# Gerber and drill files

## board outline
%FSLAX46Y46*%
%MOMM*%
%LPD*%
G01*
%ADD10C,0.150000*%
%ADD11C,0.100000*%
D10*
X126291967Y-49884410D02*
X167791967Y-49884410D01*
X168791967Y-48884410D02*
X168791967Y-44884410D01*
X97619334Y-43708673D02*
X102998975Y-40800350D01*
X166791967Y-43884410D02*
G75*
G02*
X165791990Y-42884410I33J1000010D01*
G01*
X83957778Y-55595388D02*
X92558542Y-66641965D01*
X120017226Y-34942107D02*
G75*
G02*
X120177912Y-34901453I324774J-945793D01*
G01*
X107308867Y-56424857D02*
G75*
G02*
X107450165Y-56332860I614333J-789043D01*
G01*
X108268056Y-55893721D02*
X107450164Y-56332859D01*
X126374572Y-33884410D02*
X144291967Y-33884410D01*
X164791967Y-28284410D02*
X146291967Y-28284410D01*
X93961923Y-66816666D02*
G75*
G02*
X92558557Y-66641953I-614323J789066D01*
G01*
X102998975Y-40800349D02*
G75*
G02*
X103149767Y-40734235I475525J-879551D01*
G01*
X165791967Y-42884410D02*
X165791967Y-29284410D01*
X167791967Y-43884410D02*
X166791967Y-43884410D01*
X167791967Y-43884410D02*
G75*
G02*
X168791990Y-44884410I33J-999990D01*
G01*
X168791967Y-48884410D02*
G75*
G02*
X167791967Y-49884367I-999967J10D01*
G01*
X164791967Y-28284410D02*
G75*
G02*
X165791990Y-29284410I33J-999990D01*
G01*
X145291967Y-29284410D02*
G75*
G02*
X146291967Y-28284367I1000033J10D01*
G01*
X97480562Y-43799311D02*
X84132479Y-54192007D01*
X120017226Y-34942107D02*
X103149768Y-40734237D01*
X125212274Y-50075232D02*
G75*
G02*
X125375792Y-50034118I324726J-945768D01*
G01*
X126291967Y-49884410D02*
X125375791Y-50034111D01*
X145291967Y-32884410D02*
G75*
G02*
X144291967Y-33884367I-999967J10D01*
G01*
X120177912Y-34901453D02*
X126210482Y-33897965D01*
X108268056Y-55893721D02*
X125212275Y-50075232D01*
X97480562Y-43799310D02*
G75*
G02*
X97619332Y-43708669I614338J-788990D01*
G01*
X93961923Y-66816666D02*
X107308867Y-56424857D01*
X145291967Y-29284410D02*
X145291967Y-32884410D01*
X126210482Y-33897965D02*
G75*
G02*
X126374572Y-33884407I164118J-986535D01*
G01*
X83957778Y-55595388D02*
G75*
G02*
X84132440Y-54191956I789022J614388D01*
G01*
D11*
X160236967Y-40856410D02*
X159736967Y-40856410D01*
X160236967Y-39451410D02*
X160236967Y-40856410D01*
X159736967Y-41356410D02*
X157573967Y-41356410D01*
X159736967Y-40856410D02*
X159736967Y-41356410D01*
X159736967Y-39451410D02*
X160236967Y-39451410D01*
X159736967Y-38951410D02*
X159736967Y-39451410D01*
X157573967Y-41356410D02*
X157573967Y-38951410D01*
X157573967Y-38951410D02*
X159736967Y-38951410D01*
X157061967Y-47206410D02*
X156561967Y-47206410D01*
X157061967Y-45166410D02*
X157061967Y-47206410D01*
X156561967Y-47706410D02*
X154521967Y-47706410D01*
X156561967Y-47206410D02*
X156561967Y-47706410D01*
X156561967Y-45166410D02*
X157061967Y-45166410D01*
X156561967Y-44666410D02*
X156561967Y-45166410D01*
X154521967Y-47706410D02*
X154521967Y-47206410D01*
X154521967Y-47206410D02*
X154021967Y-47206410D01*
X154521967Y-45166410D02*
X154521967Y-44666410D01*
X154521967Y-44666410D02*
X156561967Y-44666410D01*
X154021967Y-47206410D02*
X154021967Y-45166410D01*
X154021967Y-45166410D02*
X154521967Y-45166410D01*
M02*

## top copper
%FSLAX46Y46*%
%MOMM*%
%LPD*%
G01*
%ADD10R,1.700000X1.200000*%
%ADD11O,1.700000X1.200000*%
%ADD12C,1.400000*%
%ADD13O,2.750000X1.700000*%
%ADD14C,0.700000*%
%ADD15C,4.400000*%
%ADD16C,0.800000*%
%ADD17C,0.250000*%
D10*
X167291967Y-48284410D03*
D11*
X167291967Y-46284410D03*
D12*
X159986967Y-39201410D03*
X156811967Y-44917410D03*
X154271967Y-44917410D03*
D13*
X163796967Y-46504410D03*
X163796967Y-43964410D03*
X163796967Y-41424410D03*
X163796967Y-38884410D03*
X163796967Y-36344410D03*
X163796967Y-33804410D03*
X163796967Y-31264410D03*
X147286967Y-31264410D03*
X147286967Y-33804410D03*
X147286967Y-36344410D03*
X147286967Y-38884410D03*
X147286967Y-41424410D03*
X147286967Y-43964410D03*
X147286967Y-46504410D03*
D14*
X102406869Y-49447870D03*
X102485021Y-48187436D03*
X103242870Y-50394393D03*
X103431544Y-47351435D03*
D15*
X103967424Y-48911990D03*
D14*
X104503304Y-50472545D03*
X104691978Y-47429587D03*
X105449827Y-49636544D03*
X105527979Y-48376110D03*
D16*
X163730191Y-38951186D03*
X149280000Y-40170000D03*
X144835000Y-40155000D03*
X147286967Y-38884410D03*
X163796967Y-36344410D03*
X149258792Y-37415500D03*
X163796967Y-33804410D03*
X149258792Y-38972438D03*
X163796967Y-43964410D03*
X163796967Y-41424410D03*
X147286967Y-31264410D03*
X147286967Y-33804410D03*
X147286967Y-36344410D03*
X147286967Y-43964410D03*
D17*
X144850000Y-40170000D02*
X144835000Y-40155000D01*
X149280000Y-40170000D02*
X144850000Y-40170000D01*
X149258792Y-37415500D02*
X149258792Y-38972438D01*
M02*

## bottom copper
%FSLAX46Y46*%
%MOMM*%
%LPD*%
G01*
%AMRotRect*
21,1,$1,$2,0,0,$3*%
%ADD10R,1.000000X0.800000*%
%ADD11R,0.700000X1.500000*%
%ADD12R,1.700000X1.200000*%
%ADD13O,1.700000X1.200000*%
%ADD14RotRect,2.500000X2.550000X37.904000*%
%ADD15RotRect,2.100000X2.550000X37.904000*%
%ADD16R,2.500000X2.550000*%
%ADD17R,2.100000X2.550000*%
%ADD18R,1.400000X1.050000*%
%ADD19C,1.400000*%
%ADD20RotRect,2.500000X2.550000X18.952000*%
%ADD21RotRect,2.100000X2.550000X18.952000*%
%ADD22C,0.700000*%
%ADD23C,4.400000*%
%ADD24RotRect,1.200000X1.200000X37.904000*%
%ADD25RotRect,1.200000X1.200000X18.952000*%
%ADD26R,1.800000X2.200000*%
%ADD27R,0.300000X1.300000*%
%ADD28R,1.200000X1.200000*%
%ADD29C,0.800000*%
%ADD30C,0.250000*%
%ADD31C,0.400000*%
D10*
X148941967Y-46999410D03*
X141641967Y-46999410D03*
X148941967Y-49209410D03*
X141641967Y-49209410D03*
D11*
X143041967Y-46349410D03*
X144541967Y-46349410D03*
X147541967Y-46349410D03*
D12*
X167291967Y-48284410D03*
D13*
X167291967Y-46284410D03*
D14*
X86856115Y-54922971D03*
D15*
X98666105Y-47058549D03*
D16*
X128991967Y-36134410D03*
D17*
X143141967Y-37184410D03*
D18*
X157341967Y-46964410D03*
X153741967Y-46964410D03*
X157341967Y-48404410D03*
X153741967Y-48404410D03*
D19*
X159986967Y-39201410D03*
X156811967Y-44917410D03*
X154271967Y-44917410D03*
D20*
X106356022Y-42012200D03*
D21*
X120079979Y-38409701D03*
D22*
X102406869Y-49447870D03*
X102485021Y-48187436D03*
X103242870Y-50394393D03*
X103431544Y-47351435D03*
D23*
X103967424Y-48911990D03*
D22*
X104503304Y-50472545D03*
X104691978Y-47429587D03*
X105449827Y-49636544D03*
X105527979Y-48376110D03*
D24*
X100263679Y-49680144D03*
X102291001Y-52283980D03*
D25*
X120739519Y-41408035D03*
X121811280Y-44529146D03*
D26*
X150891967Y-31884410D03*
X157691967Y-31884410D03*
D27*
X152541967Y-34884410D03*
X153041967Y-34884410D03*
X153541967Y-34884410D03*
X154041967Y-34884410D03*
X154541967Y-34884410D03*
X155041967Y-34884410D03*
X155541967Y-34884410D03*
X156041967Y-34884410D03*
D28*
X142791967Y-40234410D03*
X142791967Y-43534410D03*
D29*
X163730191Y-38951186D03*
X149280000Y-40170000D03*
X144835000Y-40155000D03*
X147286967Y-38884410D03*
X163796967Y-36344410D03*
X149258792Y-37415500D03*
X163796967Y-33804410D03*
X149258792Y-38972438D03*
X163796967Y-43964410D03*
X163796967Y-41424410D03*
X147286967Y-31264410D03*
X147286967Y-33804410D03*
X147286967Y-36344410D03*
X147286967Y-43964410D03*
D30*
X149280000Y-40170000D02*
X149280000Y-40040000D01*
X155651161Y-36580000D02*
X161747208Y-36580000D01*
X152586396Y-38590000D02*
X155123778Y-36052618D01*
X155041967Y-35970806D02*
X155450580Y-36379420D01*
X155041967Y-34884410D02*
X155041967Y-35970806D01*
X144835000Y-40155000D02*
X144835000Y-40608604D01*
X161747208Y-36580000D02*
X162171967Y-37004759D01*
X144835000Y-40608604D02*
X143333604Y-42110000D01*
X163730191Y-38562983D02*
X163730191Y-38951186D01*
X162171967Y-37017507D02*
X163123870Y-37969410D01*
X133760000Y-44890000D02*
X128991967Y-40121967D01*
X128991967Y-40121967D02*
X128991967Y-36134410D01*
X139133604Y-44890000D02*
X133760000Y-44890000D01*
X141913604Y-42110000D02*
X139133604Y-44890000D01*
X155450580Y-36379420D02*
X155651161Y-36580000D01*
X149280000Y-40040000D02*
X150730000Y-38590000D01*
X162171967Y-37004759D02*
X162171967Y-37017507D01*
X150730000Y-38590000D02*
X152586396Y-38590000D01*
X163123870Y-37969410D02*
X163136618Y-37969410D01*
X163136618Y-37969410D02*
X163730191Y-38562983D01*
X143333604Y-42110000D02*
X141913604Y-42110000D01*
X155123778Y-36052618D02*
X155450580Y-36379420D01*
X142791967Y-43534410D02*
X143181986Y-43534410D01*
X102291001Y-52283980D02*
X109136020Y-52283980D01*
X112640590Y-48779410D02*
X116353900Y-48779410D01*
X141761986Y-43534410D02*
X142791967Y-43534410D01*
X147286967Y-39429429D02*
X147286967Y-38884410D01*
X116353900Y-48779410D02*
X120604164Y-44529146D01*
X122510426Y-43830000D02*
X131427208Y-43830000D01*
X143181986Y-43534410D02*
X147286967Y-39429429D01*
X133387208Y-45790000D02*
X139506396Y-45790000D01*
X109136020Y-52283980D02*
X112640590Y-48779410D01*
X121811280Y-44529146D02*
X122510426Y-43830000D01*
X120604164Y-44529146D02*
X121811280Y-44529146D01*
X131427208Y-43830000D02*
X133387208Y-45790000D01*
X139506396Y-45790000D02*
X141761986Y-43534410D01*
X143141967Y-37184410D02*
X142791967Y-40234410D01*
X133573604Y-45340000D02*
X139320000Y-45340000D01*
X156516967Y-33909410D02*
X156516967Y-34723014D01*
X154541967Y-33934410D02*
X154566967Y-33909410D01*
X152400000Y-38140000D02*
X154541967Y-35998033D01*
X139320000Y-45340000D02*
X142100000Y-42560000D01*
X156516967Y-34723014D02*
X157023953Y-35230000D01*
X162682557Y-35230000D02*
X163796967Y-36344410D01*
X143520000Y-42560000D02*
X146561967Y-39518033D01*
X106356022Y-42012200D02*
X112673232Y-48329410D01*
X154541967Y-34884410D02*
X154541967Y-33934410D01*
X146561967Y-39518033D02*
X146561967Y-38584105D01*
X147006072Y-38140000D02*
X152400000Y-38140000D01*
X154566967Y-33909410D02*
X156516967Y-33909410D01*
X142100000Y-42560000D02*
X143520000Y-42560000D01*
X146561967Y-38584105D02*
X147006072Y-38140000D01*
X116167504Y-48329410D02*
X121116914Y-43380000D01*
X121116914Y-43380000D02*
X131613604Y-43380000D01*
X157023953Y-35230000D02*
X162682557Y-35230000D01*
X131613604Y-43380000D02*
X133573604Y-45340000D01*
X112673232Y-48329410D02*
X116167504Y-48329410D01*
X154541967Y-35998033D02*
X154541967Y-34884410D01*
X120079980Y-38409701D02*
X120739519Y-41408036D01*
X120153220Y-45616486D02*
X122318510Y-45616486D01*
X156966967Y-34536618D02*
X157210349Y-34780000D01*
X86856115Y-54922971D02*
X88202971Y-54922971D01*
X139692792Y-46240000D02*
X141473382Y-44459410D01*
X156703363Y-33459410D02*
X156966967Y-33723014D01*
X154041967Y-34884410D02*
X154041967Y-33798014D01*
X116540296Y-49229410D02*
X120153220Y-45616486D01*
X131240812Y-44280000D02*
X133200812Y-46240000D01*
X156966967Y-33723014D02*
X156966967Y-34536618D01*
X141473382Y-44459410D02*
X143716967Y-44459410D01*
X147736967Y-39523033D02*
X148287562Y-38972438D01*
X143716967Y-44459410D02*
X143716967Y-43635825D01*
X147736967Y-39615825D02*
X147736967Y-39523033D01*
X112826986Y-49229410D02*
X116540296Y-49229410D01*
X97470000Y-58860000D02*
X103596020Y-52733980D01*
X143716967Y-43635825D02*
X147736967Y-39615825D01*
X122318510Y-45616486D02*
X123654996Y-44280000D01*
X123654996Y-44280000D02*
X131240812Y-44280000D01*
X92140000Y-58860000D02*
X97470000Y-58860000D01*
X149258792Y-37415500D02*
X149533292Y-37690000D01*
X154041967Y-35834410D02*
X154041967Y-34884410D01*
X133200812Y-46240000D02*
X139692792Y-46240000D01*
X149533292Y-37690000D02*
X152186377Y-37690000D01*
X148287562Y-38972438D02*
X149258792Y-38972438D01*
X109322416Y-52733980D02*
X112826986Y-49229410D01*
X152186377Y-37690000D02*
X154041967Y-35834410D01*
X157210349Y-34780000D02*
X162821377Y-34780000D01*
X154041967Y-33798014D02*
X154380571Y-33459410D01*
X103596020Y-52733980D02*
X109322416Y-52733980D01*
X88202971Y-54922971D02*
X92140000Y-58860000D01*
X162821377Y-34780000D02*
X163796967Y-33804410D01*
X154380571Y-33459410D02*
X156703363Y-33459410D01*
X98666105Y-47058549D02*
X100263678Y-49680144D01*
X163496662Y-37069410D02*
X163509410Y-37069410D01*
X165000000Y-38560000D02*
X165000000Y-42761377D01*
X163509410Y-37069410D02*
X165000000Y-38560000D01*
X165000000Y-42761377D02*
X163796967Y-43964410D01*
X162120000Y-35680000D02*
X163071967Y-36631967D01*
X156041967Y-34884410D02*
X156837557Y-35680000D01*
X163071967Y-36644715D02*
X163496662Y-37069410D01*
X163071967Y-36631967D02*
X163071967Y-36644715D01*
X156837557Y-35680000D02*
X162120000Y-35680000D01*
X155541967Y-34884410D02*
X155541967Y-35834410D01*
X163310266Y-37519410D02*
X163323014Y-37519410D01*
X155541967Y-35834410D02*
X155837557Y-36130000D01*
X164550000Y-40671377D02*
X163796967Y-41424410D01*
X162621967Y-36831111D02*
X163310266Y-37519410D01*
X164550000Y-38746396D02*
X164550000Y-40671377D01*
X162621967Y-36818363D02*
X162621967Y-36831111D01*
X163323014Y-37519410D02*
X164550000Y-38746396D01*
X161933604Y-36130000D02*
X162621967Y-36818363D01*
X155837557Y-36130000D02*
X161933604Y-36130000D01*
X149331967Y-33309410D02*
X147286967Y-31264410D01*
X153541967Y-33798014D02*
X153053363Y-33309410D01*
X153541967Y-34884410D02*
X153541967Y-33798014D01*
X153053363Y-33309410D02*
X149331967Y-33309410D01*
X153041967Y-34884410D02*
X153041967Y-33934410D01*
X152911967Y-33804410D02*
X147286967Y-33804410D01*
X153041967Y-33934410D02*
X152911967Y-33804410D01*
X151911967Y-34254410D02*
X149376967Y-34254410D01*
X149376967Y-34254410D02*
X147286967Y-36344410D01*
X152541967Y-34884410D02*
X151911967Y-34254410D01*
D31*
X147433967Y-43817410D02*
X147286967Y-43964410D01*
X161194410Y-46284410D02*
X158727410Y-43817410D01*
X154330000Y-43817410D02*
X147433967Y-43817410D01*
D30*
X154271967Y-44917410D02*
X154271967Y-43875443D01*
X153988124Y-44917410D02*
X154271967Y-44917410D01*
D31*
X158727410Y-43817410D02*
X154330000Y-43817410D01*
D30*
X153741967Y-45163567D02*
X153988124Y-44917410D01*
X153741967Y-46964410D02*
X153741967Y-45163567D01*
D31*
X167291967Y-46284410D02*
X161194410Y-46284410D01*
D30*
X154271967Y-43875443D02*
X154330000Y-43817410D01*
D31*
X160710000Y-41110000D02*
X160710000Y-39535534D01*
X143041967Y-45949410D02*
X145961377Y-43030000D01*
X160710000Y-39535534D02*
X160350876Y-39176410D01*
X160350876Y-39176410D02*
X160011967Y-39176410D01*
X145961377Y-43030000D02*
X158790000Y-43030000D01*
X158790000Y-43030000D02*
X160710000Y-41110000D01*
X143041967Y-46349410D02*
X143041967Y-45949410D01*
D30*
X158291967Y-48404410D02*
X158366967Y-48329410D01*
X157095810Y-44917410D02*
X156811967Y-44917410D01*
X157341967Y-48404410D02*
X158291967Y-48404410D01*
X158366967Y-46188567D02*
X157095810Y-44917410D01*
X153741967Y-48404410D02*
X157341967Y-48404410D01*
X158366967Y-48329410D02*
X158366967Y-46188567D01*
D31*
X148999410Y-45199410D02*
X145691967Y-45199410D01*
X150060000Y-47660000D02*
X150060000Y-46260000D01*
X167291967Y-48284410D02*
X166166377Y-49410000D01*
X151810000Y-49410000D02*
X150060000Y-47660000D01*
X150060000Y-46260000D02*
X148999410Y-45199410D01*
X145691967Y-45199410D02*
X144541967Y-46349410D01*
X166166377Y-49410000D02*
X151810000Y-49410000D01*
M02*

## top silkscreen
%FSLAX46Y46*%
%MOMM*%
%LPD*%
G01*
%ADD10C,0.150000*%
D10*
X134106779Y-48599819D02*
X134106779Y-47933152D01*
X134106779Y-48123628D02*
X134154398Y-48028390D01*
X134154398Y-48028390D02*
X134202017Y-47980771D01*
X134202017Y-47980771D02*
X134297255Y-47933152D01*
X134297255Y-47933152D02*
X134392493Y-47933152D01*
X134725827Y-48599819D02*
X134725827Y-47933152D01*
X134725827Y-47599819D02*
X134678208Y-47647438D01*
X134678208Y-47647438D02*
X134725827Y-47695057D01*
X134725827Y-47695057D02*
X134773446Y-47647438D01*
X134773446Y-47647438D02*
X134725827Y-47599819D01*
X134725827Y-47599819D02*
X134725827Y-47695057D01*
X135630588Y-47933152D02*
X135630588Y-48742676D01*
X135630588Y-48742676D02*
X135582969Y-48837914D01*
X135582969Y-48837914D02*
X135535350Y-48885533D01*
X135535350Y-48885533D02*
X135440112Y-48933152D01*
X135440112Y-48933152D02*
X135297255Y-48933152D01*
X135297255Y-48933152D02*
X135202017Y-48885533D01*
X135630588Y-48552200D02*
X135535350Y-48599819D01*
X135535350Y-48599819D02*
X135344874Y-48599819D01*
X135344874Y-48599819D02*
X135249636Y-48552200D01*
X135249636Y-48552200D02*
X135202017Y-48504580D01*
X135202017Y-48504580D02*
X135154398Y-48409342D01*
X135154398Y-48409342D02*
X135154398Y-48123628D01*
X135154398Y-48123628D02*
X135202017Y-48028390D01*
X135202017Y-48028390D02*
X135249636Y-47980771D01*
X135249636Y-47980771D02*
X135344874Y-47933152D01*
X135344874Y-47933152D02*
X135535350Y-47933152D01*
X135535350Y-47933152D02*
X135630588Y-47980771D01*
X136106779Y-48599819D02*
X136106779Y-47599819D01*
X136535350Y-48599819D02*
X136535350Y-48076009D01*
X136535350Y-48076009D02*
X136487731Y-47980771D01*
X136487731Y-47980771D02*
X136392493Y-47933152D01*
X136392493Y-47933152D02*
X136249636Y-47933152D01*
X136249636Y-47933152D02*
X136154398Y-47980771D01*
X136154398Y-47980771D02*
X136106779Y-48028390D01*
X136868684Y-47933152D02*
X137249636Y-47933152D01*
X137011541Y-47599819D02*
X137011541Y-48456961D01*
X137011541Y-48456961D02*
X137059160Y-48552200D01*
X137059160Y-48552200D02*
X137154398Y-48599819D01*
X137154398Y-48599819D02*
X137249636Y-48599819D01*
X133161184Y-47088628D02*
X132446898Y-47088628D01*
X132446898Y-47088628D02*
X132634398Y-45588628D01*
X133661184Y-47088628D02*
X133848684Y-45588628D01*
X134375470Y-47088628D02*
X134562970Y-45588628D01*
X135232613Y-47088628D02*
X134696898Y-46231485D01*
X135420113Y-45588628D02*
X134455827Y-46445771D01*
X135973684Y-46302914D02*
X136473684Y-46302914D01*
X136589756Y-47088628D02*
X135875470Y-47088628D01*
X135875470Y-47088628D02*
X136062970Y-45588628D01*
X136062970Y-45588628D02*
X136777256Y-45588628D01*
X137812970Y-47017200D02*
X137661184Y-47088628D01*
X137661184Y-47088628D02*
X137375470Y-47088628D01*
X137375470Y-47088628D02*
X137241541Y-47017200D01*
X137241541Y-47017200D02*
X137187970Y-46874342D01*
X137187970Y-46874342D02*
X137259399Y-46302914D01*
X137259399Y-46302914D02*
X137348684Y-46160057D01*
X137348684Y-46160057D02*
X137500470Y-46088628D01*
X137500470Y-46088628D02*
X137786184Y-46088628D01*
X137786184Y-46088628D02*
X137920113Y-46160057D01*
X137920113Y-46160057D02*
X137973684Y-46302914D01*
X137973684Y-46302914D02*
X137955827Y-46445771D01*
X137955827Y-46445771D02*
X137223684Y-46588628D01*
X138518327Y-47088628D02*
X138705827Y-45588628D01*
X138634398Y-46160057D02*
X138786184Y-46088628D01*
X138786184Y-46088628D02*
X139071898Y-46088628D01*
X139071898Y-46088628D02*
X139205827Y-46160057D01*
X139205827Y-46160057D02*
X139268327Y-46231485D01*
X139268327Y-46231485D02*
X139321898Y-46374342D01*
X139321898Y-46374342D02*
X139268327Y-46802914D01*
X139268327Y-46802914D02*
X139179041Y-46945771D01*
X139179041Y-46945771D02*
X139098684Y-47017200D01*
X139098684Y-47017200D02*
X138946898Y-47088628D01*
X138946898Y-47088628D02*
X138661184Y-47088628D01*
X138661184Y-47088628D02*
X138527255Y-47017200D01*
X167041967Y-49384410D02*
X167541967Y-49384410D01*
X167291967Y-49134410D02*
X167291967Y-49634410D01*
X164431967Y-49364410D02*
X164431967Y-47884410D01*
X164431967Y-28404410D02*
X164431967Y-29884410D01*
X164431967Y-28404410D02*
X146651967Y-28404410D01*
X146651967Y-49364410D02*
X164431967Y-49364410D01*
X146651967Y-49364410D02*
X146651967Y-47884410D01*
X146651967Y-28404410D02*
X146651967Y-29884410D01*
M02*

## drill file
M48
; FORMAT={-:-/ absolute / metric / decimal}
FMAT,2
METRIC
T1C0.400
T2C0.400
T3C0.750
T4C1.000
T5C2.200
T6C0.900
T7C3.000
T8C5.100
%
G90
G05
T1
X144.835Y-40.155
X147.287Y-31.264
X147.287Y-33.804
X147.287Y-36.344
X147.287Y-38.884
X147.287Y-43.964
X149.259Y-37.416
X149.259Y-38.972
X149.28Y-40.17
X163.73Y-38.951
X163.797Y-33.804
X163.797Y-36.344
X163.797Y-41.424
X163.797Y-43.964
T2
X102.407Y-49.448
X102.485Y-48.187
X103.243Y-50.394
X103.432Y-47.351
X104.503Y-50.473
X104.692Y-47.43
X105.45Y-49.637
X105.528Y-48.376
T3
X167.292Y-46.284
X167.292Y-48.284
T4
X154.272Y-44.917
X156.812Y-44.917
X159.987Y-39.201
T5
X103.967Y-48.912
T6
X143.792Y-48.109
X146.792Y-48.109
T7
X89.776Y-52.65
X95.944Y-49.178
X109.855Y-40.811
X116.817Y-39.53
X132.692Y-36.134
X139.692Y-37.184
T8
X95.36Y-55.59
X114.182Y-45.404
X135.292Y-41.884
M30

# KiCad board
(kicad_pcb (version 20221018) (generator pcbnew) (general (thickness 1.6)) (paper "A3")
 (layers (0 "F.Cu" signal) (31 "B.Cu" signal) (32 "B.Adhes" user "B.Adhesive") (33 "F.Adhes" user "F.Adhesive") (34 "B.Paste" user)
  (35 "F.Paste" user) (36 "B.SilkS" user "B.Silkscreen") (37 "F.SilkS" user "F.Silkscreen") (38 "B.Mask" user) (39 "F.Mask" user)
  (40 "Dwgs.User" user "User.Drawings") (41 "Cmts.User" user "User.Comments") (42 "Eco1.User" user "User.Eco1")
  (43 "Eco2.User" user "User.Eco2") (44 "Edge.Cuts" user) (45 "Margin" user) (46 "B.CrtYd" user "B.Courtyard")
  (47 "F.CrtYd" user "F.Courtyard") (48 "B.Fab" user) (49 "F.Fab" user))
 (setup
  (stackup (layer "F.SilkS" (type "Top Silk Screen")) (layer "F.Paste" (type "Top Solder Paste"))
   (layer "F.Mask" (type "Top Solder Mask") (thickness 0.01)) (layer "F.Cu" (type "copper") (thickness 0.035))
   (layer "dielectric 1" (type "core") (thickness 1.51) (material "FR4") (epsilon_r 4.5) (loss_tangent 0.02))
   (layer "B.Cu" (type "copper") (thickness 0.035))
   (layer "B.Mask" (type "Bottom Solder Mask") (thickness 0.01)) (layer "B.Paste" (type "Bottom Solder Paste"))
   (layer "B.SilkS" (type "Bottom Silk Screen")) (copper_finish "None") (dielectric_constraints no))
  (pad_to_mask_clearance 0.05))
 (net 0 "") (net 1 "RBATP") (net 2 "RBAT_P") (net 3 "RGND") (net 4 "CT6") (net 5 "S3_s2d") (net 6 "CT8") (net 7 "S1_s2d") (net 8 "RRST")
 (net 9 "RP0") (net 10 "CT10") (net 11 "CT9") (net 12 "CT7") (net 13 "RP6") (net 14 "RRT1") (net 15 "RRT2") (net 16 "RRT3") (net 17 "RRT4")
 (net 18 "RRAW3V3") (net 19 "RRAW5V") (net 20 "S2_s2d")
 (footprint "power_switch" (layer "F.Cu") (at 145.291967 48.08441 -90)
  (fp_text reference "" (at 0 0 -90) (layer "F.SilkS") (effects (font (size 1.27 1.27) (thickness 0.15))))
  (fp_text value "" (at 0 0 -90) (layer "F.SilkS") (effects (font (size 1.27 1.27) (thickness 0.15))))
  (pad "" smd rect (at -1.085 -3.65 180) (size 1 0.8) (layers "B.Cu" "B.Paste" "B.Mask"))
  (pad "" smd rect (at -1.085 3.65 180) (size 1 0.8) (layers "B.Cu" "B.Paste" "B.Mask"))
  (pad "" np_thru_hole circle (at 0.025 -1.5) (size 0.9 0.9) (drill 0.9) (layers "*.Cu" "*.Mask"))
  (pad "" np_thru_hole circle (at 0.025 1.5) (size 0.9 0.9) (drill 0.9) (layers "*.Cu" "*.Mask"))
  (pad "" smd rect (at 1.125 -3.65 180) (size 1 0.8) (layers "B.Cu" "B.Paste" "B.Mask"))
  (pad "" smd rect (at 1.125 3.65 180) (size 1 0.8) (layers "B.Cu" "B.Paste" "B.Mask"))
  (pad "4" smd rect (at -1.735 2.25 180) (size 0.7 1.5) (layers "B.Cu" "B.Paste" "B.Mask") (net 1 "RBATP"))
  (pad "5" smd rect (at -1.735 0.75 180) (size 0.7 1.5) (layers "B.Cu" "B.Paste" "B.Mask") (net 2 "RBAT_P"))
  (pad "6" smd rect (at -1.735 -2.25 180) (size 0.7 1.5) (layers "B.Cu" "B.Paste" "B.Mask")))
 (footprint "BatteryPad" (layer "F.Cu") (at 167.291967 47.28441 90)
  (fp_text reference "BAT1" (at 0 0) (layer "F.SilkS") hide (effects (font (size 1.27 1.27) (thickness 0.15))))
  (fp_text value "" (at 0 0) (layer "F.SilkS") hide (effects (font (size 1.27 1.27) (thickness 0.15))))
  (fp_line (start -2.1 -0.25) (end -2.1 0.25) (stroke (width 0.15) (type solid)) (layer "F.SilkS"))
  (fp_line (start -1.85 0) (end -2.35 0) (stroke (width 0.15) (type solid)) (layer "F.SilkS"))
  (pad "1" thru_hole rect (at -1 0 90) (size 1.2 1.7) (drill 0.75) (layers "*.Cu" "*.Mask") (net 2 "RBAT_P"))
  (pad "2" thru_hole oval (at 1 0 90) (size 1.2 1.7) (drill 0.75) (layers "*.Cu" "*.Mask") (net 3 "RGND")))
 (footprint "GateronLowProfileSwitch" (layer "F.Cu") (at 95.359531 55.589614 37.904)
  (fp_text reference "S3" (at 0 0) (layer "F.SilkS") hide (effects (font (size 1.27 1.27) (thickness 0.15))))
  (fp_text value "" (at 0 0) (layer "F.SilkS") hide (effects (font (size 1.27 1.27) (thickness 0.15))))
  (pad "" np_thru_hole circle (at -2.6 -5.75) (size 3 3) (drill 3) (layers "*.Cu" "*.Mask"))
  (pad "" np_thru_hole circle (at 0 0) (size 5.1 5.1) (drill 5.1) (layers "*.Cu" "*.Mask"))
  (pad "" np_thru_hole circle (at 4.4 -4.7) (size 3 3) (drill 3) (layers "*.Cu" "*.Mask"))
  (pad "1" smd rect (at -6.3 -5.75 37.904) (size 2.5 2.55) (layers "B.Cu" "B.Paste" "B.Mask") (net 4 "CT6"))
  (pad "2" smd rect (at 7.85 -4.7 37.904) (size 2.1 2.55) (layers "B.Cu" "B.Paste" "B.Mask") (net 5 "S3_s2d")))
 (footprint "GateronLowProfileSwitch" (layer "F.Cu") (at 135.291967 41.88441)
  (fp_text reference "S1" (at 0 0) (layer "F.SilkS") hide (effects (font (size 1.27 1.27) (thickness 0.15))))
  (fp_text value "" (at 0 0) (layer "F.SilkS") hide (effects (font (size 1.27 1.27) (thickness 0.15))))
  (pad "" np_thru_hole circle (at -2.6 -5.75) (size 3 3) (drill 3) (layers "*.Cu" "*.Mask"))
  (pad "" np_thru_hole circle (at 0 0) (size 5.1 5.1) (drill 5.1) (layers "*.Cu" "*.Mask"))
  (pad "" np_thru_hole circle (at 4.4 -4.7) (size 3 3) (drill 3) (layers "*.Cu" "*.Mask"))
  (pad "1" smd rect (at -6.3 -5.75) (size 2.5 2.55) (layers "B.Cu" "B.Paste" "B.Mask") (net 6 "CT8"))
  (pad "2" smd rect (at 7.85 -4.7) (size 2.1 2.55) (layers "B.Cu" "B.Paste" "B.Mask") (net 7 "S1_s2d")))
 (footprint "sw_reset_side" (layer "F.Cu") (at 155.541967 47.68441 -90)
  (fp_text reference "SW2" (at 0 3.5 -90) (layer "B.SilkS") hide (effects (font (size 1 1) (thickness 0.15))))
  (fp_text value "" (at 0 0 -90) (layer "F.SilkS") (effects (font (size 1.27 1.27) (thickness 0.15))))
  (pad "1" smd rect (at -0.72 -1.8 180) (size 1.4 1.05) (layers "B.Cu" "B.Paste" "B.Mask") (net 3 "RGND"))
  (pad "1" smd rect (at -0.72 1.8 180) (size 1.4 1.05) (layers "B.Cu" "B.Paste" "B.Mask") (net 3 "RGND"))
  (pad "2" smd rect (at 0.72 -1.8 180) (size 1.4 1.05) (layers "B.Cu" "B.Paste" "B.Mask") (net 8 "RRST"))
  (pad "2" smd rect (at 0.72 1.8 180) (size 1.4 1.05) (layers "B.Cu" "B.Paste" "B.Mask") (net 8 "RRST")))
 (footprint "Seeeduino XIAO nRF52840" (layer "F.Cu") (at 155.541967 38.88441 180)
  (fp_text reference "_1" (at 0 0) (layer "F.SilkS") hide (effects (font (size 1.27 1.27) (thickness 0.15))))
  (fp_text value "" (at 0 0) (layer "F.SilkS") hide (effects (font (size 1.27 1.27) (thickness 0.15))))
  (fp_line (start -8.89 -10.48) (end -8.89 -9) (stroke (width 0.15) (type solid)) (layer "F.SilkS"))
  (fp_line (start -8.89 10.48) (end -8.89 9) (stroke (width 0.15) (type solid)) (layer "F.SilkS"))
  (fp_line (start -8.89 10.48) (end 8.89 10.48) (stroke (width 0.15) (type solid)) (layer "F.SilkS"))
  (fp_line (start 8.89 -10.48) (end -8.89 -10.48) (stroke (width 0.15) (type solid)) (layer "F.SilkS"))
  (fp_line (start 8.89 -10.48) (end 8.89 -9) (stroke (width 0.15) (type solid)) (layer "F.SilkS"))
  (fp_line (start 8.89 10.48) (end 8.89 9) (stroke (width 0.15) (type solid)) (layer "F.SilkS"))
  (fp_line (start -4.695 -1.972) (end -4.195 -1.972) (stroke (width 0.1) (type solid)) (layer "Edge.Cuts"))
  (fp_line (start -4.695 -0.567) (end -4.695 -1.972) (stroke (width 0.1) (type solid)) (layer "Edge.Cuts"))
  (fp_line (start -4.195 -2.472) (end -2.032 -2.472) (stroke (width 0.1) (type solid)) (layer "Edge.Cuts"))
  (fp_line (start -4.195 -1.972) (end -4.195 -2.472) (stroke (width 0.1) (type solid)) (layer "Edge.Cuts"))
  (fp_line (start -4.195 -0.567) (end -4.695 -0.567) (stroke (width 0.1) (type solid)) (layer "Edge.Cuts"))
  (fp_line (start -4.195 -0.067) (end -4.195 -0.567) (stroke (width 0.1) (type solid)) (layer "Edge.Cuts"))
  (fp_line (start -2.032 -2.472) (end -2.032 -0.067) (stroke (width 0.1) (type solid)) (layer "Edge.Cuts"))
  (fp_line (start -2.032 -0.067) (end -4.195 -0.067) (stroke (width 0.1) (type solid)) (layer "Edge.Cuts"))
  (fp_line (start -1.52 -8.322) (end -1.02 -8.322) (stroke (width 0.1) (type solid)) (layer "Edge.Cuts"))
  (fp_line (start -1.52 -6.282) (end -1.52 -8.322) (stroke (width 0.1) (type solid)) (layer "Edge.Cuts"))
  (fp_line (start -1.02 -8.822) (end 1.02 -8.822) (stroke (width 0.1) (type solid)) (layer "Edge.Cuts"))
  (fp_line (start -1.02 -8.322) (end -1.02 -8.822) (stroke (width 0.1) (type solid)) (layer "Edge.Cuts"))
  (fp_line (start -1.02 -6.282) (end -1.52 -6.282) (stroke (width 0.1) (type solid)) (layer "Edge.Cuts"))
  (fp_line (start -1.02 -5.782) (end -1.02 -6.282) (stroke (width 0.1) (type solid)) (layer "Edge.Cuts"))
  (fp_line (start 1.02 -8.822) (end 1.02 -8.322) (stroke (width 0.1) (type solid)) (layer "Edge.Cuts"))
  (fp_line (start 1.02 -8.322) (end 1.52 -8.322) (stroke (width 0.1) (type solid)) (layer "Edge.Cuts"))
  (fp_line (start 1.02 -6.282) (end 1.02 -5.782) (stroke (width 0.1) (type solid)) (layer "Edge.Cuts"))
  (fp_line (start 1.02 -5.782) (end -1.02 -5.782) (stroke (width 0.1) (type solid)) (layer "Edge.Cuts"))
  (fp_line (start 1.52 -8.322) (end 1.52 -6.282) (stroke (width 0.1) (type solid)) (layer "Edge.Cuts"))
  (fp_line (start 1.52 -6.282) (end 1.02 -6.282) (stroke (width 0.1) (type solid)) (layer "Edge.Cuts"))
  (pad "" thru_hole circle (at -4.445 -0.317) (size 1.4 1.4) (drill 1) (layers "*.Cu" "*.Mask") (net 1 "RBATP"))
  (pad "" thru_hole circle (at -1.27 -6.033) (size 1.4 1.4) (drill 1) (layers "*.Cu" "*.Mask") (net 8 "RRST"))
  (pad "" thru_hole circle (at 1.27 -6.033) (size 1.4 1.4) (drill 1) (layers "*.Cu" "*.Mask") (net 3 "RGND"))
  (pad "1" smd oval (at -8.255 -7.62 180) (size 2.75 1.7) (layers "F.Cu" "F.Paste" "F.Mask") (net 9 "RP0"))
  (pad "2" smd oval (at -8.255 -5.08 180) (size 2.75 1.7) (layers "F.Cu" "F.Paste" "F.Mask") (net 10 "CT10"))
  (pad "3" smd oval (at -8.255 -2.54 180) (size 2.75 1.7) (layers "F.Cu" "F.Paste" "F.Mask") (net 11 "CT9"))
  (pad "4" smd oval (at -8.255 0 180) (size 2.75 1.7) (layers "F.Cu" "F.Paste" "F.Mask") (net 6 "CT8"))
  (pad "5" smd oval (at -8.255 2.54 180) (size 2.75 1.7) (layers "F.Cu" "F.Paste" "F.Mask") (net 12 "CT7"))
  (pad "6" smd oval (at -8.255 5.08 180) (size 2.75 1.7) (layers "F.Cu" "F.Paste" "F.Mask") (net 4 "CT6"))
  (pad "7" smd oval (at -8.255 7.62 180) (size 2.75 1.7) (layers "F.Cu" "F.Paste" "F.Mask") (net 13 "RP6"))
  (pad "8" smd oval (at 8.255 7.62 180) (size 2.75 1.7) (layers "F.Cu" "F.Paste" "F.Mask") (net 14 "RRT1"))
  (pad "9" smd oval (at 8.255 5.08 180) (size 2.75 1.7) (layers "F.Cu" "F.Paste" "F.Mask") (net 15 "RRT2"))
  (pad "10" smd oval (at 8.255 2.54 180) (size 2.75 1.7) (layers "F.Cu" "F.Paste" "F.Mask") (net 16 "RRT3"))
  (pad "11" smd oval (at 8.255 0 180) (size 2.75 1.7) (layers "F.Cu" "F.Paste" "F.Mask") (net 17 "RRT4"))
  (pad "12" smd oval (at 8.255 -2.54 180) (size 2.75 1.7) (layers "F.Cu" "F.Paste" "F.Mask") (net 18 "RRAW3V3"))
  (pad "13" smd oval (at 8.255 -5.08 180) (size 2.75 1.7) (layers "F.Cu" "F.Paste" "F.Mask") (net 3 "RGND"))
  (pad "14" smd oval (at 8.255 -7.62 180) (size 2.75 1.7) (layers "F.Cu" "F.Paste" "F.Mask") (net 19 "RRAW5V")))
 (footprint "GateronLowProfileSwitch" (layer "F.Cu") (at 114.181967 45.40441 18.952)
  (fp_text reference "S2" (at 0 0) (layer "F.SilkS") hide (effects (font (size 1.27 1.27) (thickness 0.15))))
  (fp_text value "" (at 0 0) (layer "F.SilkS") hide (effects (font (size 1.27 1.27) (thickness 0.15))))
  (pad "" np_thru_hole circle (at -2.6 -5.75) (size 3 3) (drill 3) (layers "*.Cu" "*.Mask"))
  (pad "" np_thru_hole circle (at 0 0) (size 5.1 5.1) (drill 5.1) (layers "*.Cu" "*.Mask"))
  (pad "" np_thru_hole circle (at 4.4 -4.7) (size 3 3) (drill 3) (layers "*.Cu" "*.Mask"))
  (pad "1" smd rect (at -6.3 -5.75 18.952) (size 2.5 2.55) (layers "B.Cu" "B.Paste" "B.Mask") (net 12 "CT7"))
  (pad "2" smd rect (at 7.85 -4.7 18.952) (size 2.1 2.55) (layers "B.Cu" "B.Paste" "B.Mask") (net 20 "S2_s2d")))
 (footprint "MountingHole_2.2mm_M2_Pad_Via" (layer "F.Cu") (at 103.967424 48.91199 18.952)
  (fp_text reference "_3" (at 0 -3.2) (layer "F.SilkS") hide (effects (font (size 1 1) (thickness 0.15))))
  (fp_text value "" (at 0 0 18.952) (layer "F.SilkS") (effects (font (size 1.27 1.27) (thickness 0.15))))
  (pad "1" thru_hole circle (at -1.65 0) (size 0.7 0.7) (drill 0.4) (layers "*.Cu" "*.Mask"))
  (pad "1" thru_hole circle (at -1.166726 -1.166726) (size 0.7 0.7) (drill 0.4) (layers "*.Cu" "*.Mask"))
  (pad "1" thru_hole circle (at -1.166726 1.166726) (size 0.7 0.7) (drill 0.4) (layers "*.Cu" "*.Mask"))
  (pad "1" thru_hole circle (at 0 -1.65) (size 0.7 0.7) (drill 0.4) (layers "*.Cu" "*.Mask"))
  (pad "1" thru_hole circle (at 0 0) (size 4.4 4.4) (drill 2.2) (layers "*.Cu" "*.Mask"))
  (pad "1" thru_hole circle (at 0 1.65) (size 0.7 0.7) (drill 0.4) (layers "*.Cu" "*.Mask"))
  (pad "1" thru_hole circle (at 1.166726 -1.166726) (size 0.7 0.7) (drill 0.4) (layers "*.Cu" "*.Mask"))
  (pad "1" thru_hole circle (at 1.166726 1.166726) (size 0.7 0.7) (drill 0.4) (layers "*.Cu" "*.Mask"))
  (pad "1" thru_hole circle (at 1.65 0) (size 0.7 0.7) (drill 0.4) (layers "*.Cu" "*.Mask")))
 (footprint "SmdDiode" (layer "B.Cu") (at 95.359531 55.589614 37.904)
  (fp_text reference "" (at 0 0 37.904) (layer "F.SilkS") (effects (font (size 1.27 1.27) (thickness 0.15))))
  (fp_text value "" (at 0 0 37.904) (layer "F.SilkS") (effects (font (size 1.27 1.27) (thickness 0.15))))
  (pad "1" smd rect (at 7.5 -1.65 37.904) (size 1.2 1.2) (layers "B.Cu" "B.Paste" "B.Mask") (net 5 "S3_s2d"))
  (pad "2" smd rect (at 7.5 1.65 37.904) (size 1.2 1.2) (layers "B.Cu" "B.Paste" "B.Mask") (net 17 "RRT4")))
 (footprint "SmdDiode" (layer "B.Cu") (at 114.181967 45.40441 18.952)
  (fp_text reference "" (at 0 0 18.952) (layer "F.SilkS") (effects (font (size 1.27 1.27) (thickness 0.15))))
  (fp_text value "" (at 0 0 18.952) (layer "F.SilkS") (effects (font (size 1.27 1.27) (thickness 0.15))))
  (pad "1" smd rect (at 7.5 -1.65 18.952) (size 1.2 1.2) (layers "B.Cu" "B.Paste" "B.Mask") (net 20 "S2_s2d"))
  (pad "2" smd rect (at 7.5 1.65 18.952) (size 1.2 1.2) (layers "B.Cu" "B.Paste" "B.Mask") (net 17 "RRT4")))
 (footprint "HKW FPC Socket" (layer "B.Cu") (at 154.291967 31.88441)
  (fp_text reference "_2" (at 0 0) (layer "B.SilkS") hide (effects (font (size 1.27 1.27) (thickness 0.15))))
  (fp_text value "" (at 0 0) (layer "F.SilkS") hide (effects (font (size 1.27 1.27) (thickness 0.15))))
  (pad "" smd rect (at -3.4 0) (size 1.8 2.2) (layers "B.Cu" "B.Paste" "B.Mask"))
  (pad "" smd rect (at 3.4 0) (size 1.8 2.2) (layers "B.Cu" "B.Paste" "B.Mask"))
  (pad "1" smd rect (at -1.75 3) (size 0.3 1.3) (layers "B.Cu" "B.Paste" "B.Mask") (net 16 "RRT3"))
  (pad "2" smd rect (at -1.25 3) (size 0.3 1.3) (layers "B.Cu" "B.Paste" "B.Mask") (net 15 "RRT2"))
  (pad "3" smd rect (at -0.75 3) (size 0.3 1.3) (layers "B.Cu" "B.Paste" "B.Mask") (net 14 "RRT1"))
  (pad "4" smd rect (at -0.25 3) (size 0.3 1.3) (layers "B.Cu" "B.Paste" "B.Mask") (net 4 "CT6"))
  (pad "5" smd rect (at 0.25 3) (size 0.3 1.3) (layers "B.Cu" "B.Paste" "B.Mask") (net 12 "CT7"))
  (pad "6" smd rect (at 0.75 3) (size 0.3 1.3) (layers "B.Cu" "B.Paste" "B.Mask") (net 6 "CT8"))
  (pad "7" smd rect (at 1.25 3) (size 0.3 1.3) (layers "B.Cu" "B.Paste" "B.Mask") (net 11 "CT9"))
  (pad "8" smd rect (at 1.75 3) (size 0.3 1.3) (layers "B.Cu" "B.Paste" "B.Mask") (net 10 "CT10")))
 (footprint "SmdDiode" (layer "B.Cu") (at 135.291967 41.88441)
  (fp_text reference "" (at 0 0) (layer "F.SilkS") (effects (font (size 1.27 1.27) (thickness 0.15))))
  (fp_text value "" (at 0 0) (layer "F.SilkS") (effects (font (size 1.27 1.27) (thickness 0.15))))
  (pad "1" smd rect (at 7.5 -1.65) (size 1.2 1.2) (layers "B.Cu" "B.Paste" "B.Mask") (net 7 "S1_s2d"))
  (pad "2" smd rect (at 7.5 1.65) (size 1.2 1.2) (layers "B.Cu" "B.Paste" "B.Mask") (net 17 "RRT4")))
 (gr_line (start 126.291967 49.88441) (end 167.791967 49.88441) (stroke (width 0.15) (type solid)) (layer "Edge.Cuts"))
 (gr_line (start 168.791967 48.88441) (end 168.791967 44.88441) (stroke (width 0.15) (type solid)) (layer "Edge.Cuts"))
 (gr_line (start 97.619334 43.708673) (end 102.998975 40.80035) (stroke (width 0.15) (type solid)) (layer "Edge.Cuts"))
 (gr_arc (start 166.791967 43.88441) (mid 166.08486 43.591517) (end 165.791967 42.88441) (stroke (width 0.15) (type solid))
  (layer "Edge.Cuts"))
 (gr_line (start 83.957778 55.595388) (end 92.558542 66.641965) (stroke (width 0.15) (type solid)) (layer "Edge.Cuts"))
 (gr_arc (start 120.017226 34.942107) (mid 120.096725 34.918445) (end 120.177912 34.901453) (stroke (width 0.15) (type solid))
  (layer "Edge.Cuts"))
 (gr_arc (start 107.308867 56.424857) (mid 107.377573 56.375875) (end 107.450164 56.332859) (stroke (width 0.15) (type solid))
  (layer "Edge.Cuts"))
 (gr_line (start 108.268056 55.893721) (end 107.450164 56.332859) (stroke (width 0.15) (type solid)) (layer "Edge.Cuts"))
 (gr_line (start 126.374572 33.88441) (end 144.291967 33.88441) (stroke (width 0.15) (type solid)) (layer "Edge.Cuts"))
 (gr_line (start 164.791967 28.28441) (end 146.291967 28.28441) (stroke (width 0.15) (type solid)) (layer "Edge.Cuts"))
 (gr_arc (start 93.961923 66.816666) (mid 93.224051 67.019965) (end 92.558542 66.641965) (stroke (width 0.15) (type solid))
  (layer "Edge.Cuts"))
 (gr_arc (start 102.998975 40.800349) (mid 103.073008 40.764184) (end 103.149768 40.734237) (stroke (width 0.15) (type solid))
  (layer "Edge.Cuts"))
 (gr_line (start 165.791967 42.88441) (end 165.791967 29.28441) (stroke (width 0.15) (type solid)) (layer "Edge.Cuts"))
 (gr_line (start 167.791967 43.88441) (end 166.791967 43.88441) (stroke (width 0.15) (type solid)) (layer "Edge.Cuts"))
 (gr_arc (start 167.791967 43.88441) (mid 168.499074 44.177303) (end 168.791967 44.88441) (stroke (width 0.15) (type solid))
  (layer "Edge.Cuts"))
 (gr_arc (start 168.791967 48.88441) (mid 168.499074 49.591517) (end 167.791967 49.88441) (stroke (width 0.15) (type solid))
  (layer "Edge.Cuts"))
 (gr_arc (start 164.791967 28.28441) (mid 165.499074 28.577303) (end 165.791967 29.28441) (stroke (width 0.15) (type solid))
  (layer "Edge.Cuts"))
 (gr_arc (start 145.291967 29.28441) (mid 145.58486 28.577303) (end 146.291967 28.28441) (stroke (width 0.15) (type solid))
  (layer "Edge.Cuts"))
 (gr_line (start 97.480562 43.799311) (end 84.132479 54.192007) (stroke (width 0.15) (type solid)) (layer "Edge.Cuts"))
 (gr_line (start 120.017226 34.942107) (end 103.149768 40.734237) (stroke (width 0.15) (type solid)) (layer "Edge.Cuts"))
 (gr_arc (start 125.212274 50.075232) (mid 125.293164 50.051219) (end 125.375791 50.034111) (stroke (width 0.15) (type solid))
  (layer "Edge.Cuts"))
 (gr_line (start 126.291967 49.88441) (end 125.375791 50.034111) (stroke (width 0.15) (type solid)) (layer "Edge.Cuts"))
 (gr_arc (start 145.291967 32.88441) (mid 144.999074 33.591517) (end 144.291967 33.88441) (stroke (width 0.15) (type solid))
  (layer "Edge.Cuts"))
 (gr_line (start 120.177912 34.901453) (end 126.210482 33.897965) (stroke (width 0.15) (type solid)) (layer "Edge.Cuts"))
 (gr_line (start 108.268056 55.893721) (end 125.212275 50.075232) (stroke (width 0.15) (type solid)) (layer "Edge.Cuts"))
 (gr_arc (start 97.480562 43.79931) (mid 97.548067 43.751111) (end 97.619334 43.708673) (stroke (width 0.15) (type solid))
  (layer "Edge.Cuts"))
 (gr_line (start 93.961923 66.816666) (end 107.308867 56.424857) (stroke (width 0.15) (type solid)) (layer "Edge.Cuts"))
 (gr_line (start 145.291967 29.28441) (end 145.291967 32.88441) (stroke (width 0.15) (type solid)) (layer "Edge.Cuts"))
 (gr_arc (start 126.210482 33.897965) (mid 126.292248 33.887805) (end 126.374572 33.88441) (stroke (width 0.15) (type solid))
  (layer "Edge.Cuts"))
 (gr_arc (start 83.957778 55.595388) (mid 83.754479 54.857516) (end 84.132479 54.192007) (stroke (width 0.15) (type solid))
  (layer "Edge.Cuts"))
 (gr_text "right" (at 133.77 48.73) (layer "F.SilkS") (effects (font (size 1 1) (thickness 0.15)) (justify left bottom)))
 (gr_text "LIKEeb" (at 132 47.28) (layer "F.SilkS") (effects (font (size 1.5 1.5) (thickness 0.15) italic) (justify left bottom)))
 (segment (start 144.85 40.17) (end 144.835 40.155) (width 0.25) (layer "F.Cu") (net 6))
 (segment (start 149.28 40.17) (end 144.85 40.17) (width 0.25) (layer "F.Cu") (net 6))
 (via (at 163.730191 38.951186) (size 0.8) (drill 0.4) (layers "F.Cu" "B.Cu") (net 6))
 (via (at 149.28 40.17) (size 0.8) (drill 0.4) (layers "F.Cu" "B.Cu") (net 6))
 (via (at 144.835 40.155) (size 0.8) (drill 0.4) (layers "F.Cu" "B.Cu") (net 6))
 (segment (start 149.28 40.17) (end 149.28 40.04) (width 0.25) (layer "B.Cu") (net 6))
 (segment (start 155.651161 36.58) (end 161.747208 36.58) (width 0.25) (layer "B.Cu") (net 6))
 (segment (start 152.586396 38.59) (end 155.123778 36.052618) (width 0.25) (layer "B.Cu") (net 6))
 (segment (start 155.041967 35.970806) (end 155.45058 36.37942) (width 0.25) (layer "B.Cu") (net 6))
 (segment (start 155.041967 34.88441) (end 155.041967 35.970806) (width 0.25) (layer "B.Cu") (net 6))
 (segment (start 144.835 40.155) (end 144.835 40.608604) (width 0.25) (layer "B.Cu") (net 6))
 (segment (start 161.747208 36.58) (end 162.171967 37.004759) (width 0.25) (layer "B.Cu") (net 6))
 (segment (start 144.835 40.608604) (end 143.333604 42.11) (width 0.25) (layer "B.Cu") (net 6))
 (segment (start 163.730191 38.562983) (end 163.730191 38.951186) (width 0.25) (layer "B.Cu") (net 6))
 (segment (start 162.171967 37.017507) (end 163.12387 37.96941) (width 0.25) (layer "B.Cu") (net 6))
 (segment (start 133.76 44.89) (end 128.991967 40.121967) (width 0.25) (layer "B.Cu") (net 6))
 (segment (start 128.991967 40.121967) (end 128.991967 36.13441) (width 0.25) (layer "B.Cu") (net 6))
 (segment (start 139.133604 44.89) (end 133.76 44.89) (width 0.25) (layer "B.Cu") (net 6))
 (segment (start 141.913604 42.11) (end 139.133604 44.89) (width 0.25) (layer "B.Cu") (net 6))
 (segment (start 155.45058 36.37942) (end 155.651161 36.58) (width 0.25) (layer "B.Cu") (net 6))
 (segment (start 149.28 40.04) (end 150.73 38.59) (width 0.25) (layer "B.Cu") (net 6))
 (segment (start 162.171967 37.004759) (end 162.171967 37.017507) (width 0.25) (layer "B.Cu") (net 6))
 (segment (start 150.73 38.59) (end 152.586396 38.59) (width 0.25) (layer "B.Cu") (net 6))
 (segment (start 163.12387 37.96941) (end 163.136618 37.96941) (width 0.25) (layer "B.Cu") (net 6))
 (segment (start 163.136618 37.96941) (end 163.730191 38.562983) (width 0.25) (layer "B.Cu") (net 6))
 (segment (start 143.333604 42.11) (end 141.913604 42.11) (width 0.25) (layer "B.Cu") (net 6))
 (segment (start 155.123778 36.052618) (end 155.45058 36.37942) (width 0.25) (layer "B.Cu") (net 6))
 (via (at 147.286967 38.88441) (size 0.8) (drill 0.4) (layers "F.Cu" "B.Cu") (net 17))
 (segment (start 142.791967 43.53441) (end 143.181986 43.53441) (width 0.25) (layer "B.Cu") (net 17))
 (segment (start 102.291001 52.28398) (end 109.13602 52.28398) (width 0.25) (layer "B.Cu") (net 17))
 (segment (start 112.64059 48.77941) (end 116.3539 48.77941) (width 0.25) (layer "B.Cu") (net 17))
 (segment (start 141.761986 43.53441) (end 142.791967 43.53441) (width 0.25) (layer "B.Cu") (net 17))
 (segment (start 147.286967 39.429429) (end 147.286967 38.88441) (width 0.25) (layer "B.Cu") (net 17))
 (segment (start 116.3539 48.77941) (end 120.604164 44.529146) (width 0.25) (layer "B.Cu") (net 17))
 (segment (start 122.510426 43.83) (end 131.427208 43.83) (width 0.25) (layer "B.Cu") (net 17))
 (segment (start 143.181986 43.53441) (end 147.286967 39.429429) (width 0.25) (layer "B.Cu") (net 17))
 (segment (start 133.387208 45.79) (end 139.506396 45.79) (width 0.25) (layer "B.Cu") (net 17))
 (segment (start 109.13602 52.28398) (end 112.64059 48.77941) (width 0.25) (layer "B.Cu") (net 17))
 (segment (start 121.81128 44.529146) (end 122.510426 43.83) (width 0.25) (layer "B.Cu") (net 17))
 (segment (start 120.604164 44.529146) (end 121.81128 44.529146) (width 0.25) (layer "B.Cu") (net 17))
 (segment (start 131.427208 43.83) (end 133.387208 45.79) (width 0.25) (layer "B.Cu") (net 17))
 (segment (start 139.506396 45.79) (end 141.761986 43.53441) (width 0.25) (layer "B.Cu") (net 17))
 (segment (start 143.141967 37.18441) (end 142.791967 40.23441) (width 0.25) (layer "B.Cu") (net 7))
 (via (at 163.796967 36.34441) (size 0.8) (drill 0.4) (layers "F.Cu" "B.Cu") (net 12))
 (segment (start 133.573604 45.34) (end 139.32 45.34) (width 0.25) (layer "B.Cu") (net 12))
 (segment (start 156.516967 33.90941) (end 156.516967 34.723014) (width 0.25) (layer "B.Cu") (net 12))
 (segment (start 154.541967 33.93441) (end 154.566967 33.90941) (width 0.25) (layer "B.Cu") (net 12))
 (segment (start 152.4 38.14) (end 154.541967 35.998033) (width 0.25) (layer "B.Cu") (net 12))
 (segment (start 139.32 45.34) (end 142.1 42.56) (width 0.25) (layer "B.Cu") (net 12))
 (segment (start 156.516967 34.723014) (end 157.023953 35.23) (width 0.25) (layer "B.Cu") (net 12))
 (segment (start 162.682557 35.23) (end 163.796967 36.34441) (width 0.25) (layer "B.Cu") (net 12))
 (segment (start 143.52 42.56) (end 146.561967 39.518033) (width 0.25) (layer "B.Cu") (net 12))
 (segment (start 106.356022 42.0122) (end 112.673232 48.32941) (width 0.25) (layer "B.Cu") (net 12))
 (segment (start 154.541967 34.88441) (end 154.541967 33.93441) (width 0.25) (layer "B.Cu") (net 12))
 (segment (start 146.561967 39.518033) (end 146.561967 38.584105) (width 0.25) (layer "B.Cu") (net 12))
 (segment (start 147.006072 38.14) (end 152.4 38.14) (width 0.25) (layer "B.Cu") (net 12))
 (segment (start 154.566967 33.90941) (end 156.516967 33.90941) (width 0.25) (layer "B.Cu") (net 12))
 (segment (start 142.1 42.56) (end 143.52 42.56) (width 0.25) (layer "B.Cu") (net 12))
 (segment (start 146.561967 38.584105) (end 147.006072 38.14) (width 0.25) (layer "B.Cu") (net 12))
 (segment (start 116.167504 48.32941) (end 121.116914 43.38) (width 0.25) (layer "B.Cu") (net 12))
 (segment (start 121.116914 43.38) (end 131.613604 43.38) (width 0.25) (layer "B.Cu") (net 12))
 (segment (start 157.023953 35.23) (end 162.682557 35.23) (width 0.25) (layer "B.Cu") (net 12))
 (segment (start 131.613604 43.38) (end 133.573604 45.34) (width 0.25) (layer "B.Cu") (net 12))
 (segment (start 112.673232 48.32941) (end 116.167504 48.32941) (width 0.25) (layer "B.Cu") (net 12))
 (segment (start 154.541967 35.998033) (end 154.541967 34.88441) (width 0.25) (layer "B.Cu") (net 12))
 (segment (start 120.07998 38.409701) (end 120.739519 41.408036) (width 0.25) (layer "B.Cu") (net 20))
 (segment (start 149.258792 37.4155) (end 149.258792 38.972438) (width 0.25) (layer "F.Cu") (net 4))
 (via (at 149.258792 37.4155) (size 0.8) (drill 0.4) (layers "F.Cu" "B.Cu") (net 4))
 (via (at 163.796967 33.80441) (size 0.8) (drill 0.4) (layers "F.Cu" "B.Cu") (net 4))
 (via (at 149.258792 38.972438) (size 0.8) (drill 0.4) (layers "F.Cu" "B.Cu") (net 4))
 (segment (start 120.15322 45.616486) (end 122.31851 45.616486) (width 0.25) (layer "B.Cu") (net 4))
 (segment (start 156.966967 34.536618) (end 157.210349 34.78) (width 0.25) (layer "B.Cu") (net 4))
 (segment (start 86.856115 54.922971) (end 88.202971 54.922971) (width 0.25) (layer "B.Cu") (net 4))
 (segment (start 139.692792 46.24) (end 141.473382 44.45941) (width 0.25) (layer "B.Cu") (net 4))
 (segment (start 156.703363 33.45941) (end 156.966967 33.723014) (width 0.25) (layer "B.Cu") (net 4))
 (segment (start 154.041967 34.88441) (end 154.041967 33.798014) (width 0.25) (layer "B.Cu") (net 4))
 (segment (start 116.540296 49.22941) (end 120.15322 45.616486) (width 0.25) (layer "B.Cu") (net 4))
 (segment (start 131.240812 44.28) (end 133.200812 46.24) (width 0.25) (layer "B.Cu") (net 4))
 (segment (start 156.966967 33.723014) (end 156.966967 34.536618) (width 0.25) (layer "B.Cu") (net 4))
 (segment (start 141.473382 44.45941) (end 143.716967 44.45941) (width 0.25) (layer "B.Cu") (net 4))
 (segment (start 147.736967 39.523033) (end 148.287562 38.972438) (width 0.25) (layer "B.Cu") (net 4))
 (segment (start 143.716967 44.45941) (end 143.716967 43.635825) (width 0.25) (layer "B.Cu") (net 4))
 (segment (start 147.736967 39.615825) (end 147.736967 39.523033) (width 0.25) (layer "B.Cu") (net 4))
 (segment (start 112.826986 49.22941) (end 116.540296 49.22941) (width 0.25) (layer "B.Cu") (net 4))
 (segment (start 97.47 58.86) (end 103.59602 52.73398) (width 0.25) (layer "B.Cu") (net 4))
 (segment (start 143.716967 43.635825) (end 147.736967 39.615825) (width 0.25) (layer "B.Cu") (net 4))
 (segment (start 122.31851 45.616486) (end 123.654996 44.28) (width 0.25) (layer "B.Cu") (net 4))
 (segment (start 123.654996 44.28) (end 131.240812 44.28) (width 0.25) (layer "B.Cu") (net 4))
 (segment (start 92.14 58.86) (end 97.47 58.86) (width 0.25) (layer "B.Cu") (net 4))
 (segment (start 149.258792 37.4155) (end 149.533292 37.69) (width 0.25) (layer "B.Cu") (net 4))
 (segment (start 154.041967 35.83441) (end 154.041967 34.88441) (width 0.25) (layer "B.Cu") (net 4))
 (segment (start 133.200812 46.24) (end 139.692792 46.24) (width 0.25) (layer "B.Cu") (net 4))
 (segment (start 149.533292 37.69) (end 152.186377 37.69) (width 0.25) (layer "B.Cu") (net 4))
 (segment (start 148.287562 38.972438) (end 149.258792 38.972438) (width 0.25) (layer "B.Cu") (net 4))
 (segment (start 109.322416 52.73398) (end 112.826986 49.22941) (width 0.25) (layer "B.Cu") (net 4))
 (segment (start 152.186377 37.69) (end 154.041967 35.83441) (width 0.25) (layer "B.Cu") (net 4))
 (segment (start 157.210349 34.78) (end 162.821377 34.78) (width 0.25) (layer "B.Cu") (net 4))
 (segment (start 154.041967 33.798014) (end 154.380571 33.45941) (width 0.25) (layer "B.Cu") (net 4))
 (segment (start 103.59602 52.73398) (end 109.322416 52.73398) (width 0.25) (layer "B.Cu") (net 4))
 (segment (start 88.202971 54.922971) (end 92.14 58.86) (width 0.25) (layer "B.Cu") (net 4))
 (segment (start 162.821377 34.78) (end 163.796967 33.80441) (width 0.25) (layer "B.Cu") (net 4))
 (segment (start 154.380571 33.45941) (end 156.703363 33.45941) (width 0.25) (layer "B.Cu") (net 4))
 (segment (start 98.666105 47.058549) (end 100.263678 49.680144) (width 0.25) (layer "B.Cu") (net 5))
 (via (at 163.796967 43.96441) (size 0.8) (drill 0.4) (layers "F.Cu" "B.Cu") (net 10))
 (segment (start 163.496662 37.06941) (end 163.50941 37.06941) (width 0.25) (layer "B.Cu") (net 10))
 (segment (start 165 38.56) (end 165 42.761377) (width 0.25) (layer "B.Cu") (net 10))
 (segment (start 163.50941 37.06941) (end 165 38.56) (width 0.25) (layer "B.Cu") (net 10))
 (segment (start 165 42.761377) (end 163.796967 43.96441) (width 0.25) (layer "B.Cu") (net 10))
 (segment (start 162.12 35.68) (end 163.071967 36.631967) (width 0.25) (layer "B.Cu") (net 10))
 (segment (start 156.041967 34.88441) (end 156.837557 35.68) (width 0.25) (layer "B.Cu") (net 10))
 (segment (start 163.071967 36.644715) (end 163.496662 37.06941) (width 0.25) (layer "B.Cu") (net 10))
 (segment (start 163.071967 36.631967) (end 163.071967 36.644715) (width 0.25) (layer "B.Cu") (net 10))
 (segment (start 156.837557 35.68) (end 162.12 35.68) (width 0.25) (layer "B.Cu") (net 10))
 (via (at 163.796967 41.42441) (size 0.8) (drill 0.4) (layers "F.Cu" "B.Cu") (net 11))
 (segment (start 155.541967 34.88441) (end 155.541967 35.83441) (width 0.25) (layer "B.Cu") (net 11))
 (segment (start 163.310266 37.51941) (end 163.323014 37.51941) (width 0.25) (layer "B.Cu") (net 11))
 (segment (start 155.541967 35.83441) (end 155.837557 36.13) (width 0.25) (layer "B.Cu") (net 11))
 (segment (start 164.55 40.671377) (end 163.796967 41.42441) (width 0.25) (layer "B.Cu") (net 11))
 (segment (start 162.621967 36.831111) (end 163.310266 37.51941) (width 0.25) (layer "B.Cu") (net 11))
 (segment (start 164.55 38.746396) (end 164.55 40.671377) (width 0.25) (layer "B.Cu") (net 11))
 (segment (start 162.621967 36.818363) (end 162.621967 36.831111) (width 0.25) (layer "B.Cu") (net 11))
 (segment (start 163.323014 37.51941) (end 164.55 38.746396) (width 0.25) (layer "B.Cu") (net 11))
 (segment (start 161.933604 36.13) (end 162.621967 36.818363) (width 0.25) (layer "B.Cu") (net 11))
 (segment (start 155.837557 36.13) (end 161.933604 36.13) (width 0.25) (layer "B.Cu") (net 11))
 (via (at 147.286967 31.26441) (size 0.8) (drill 0.4) (layers "F.Cu" "B.Cu") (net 14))
 (segment (start 149.331967 33.30941) (end 147.286967 31.26441) (width 0.25) (layer "B.Cu") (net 14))
 (segment (start 153.541967 33.798014) (end 153.053363 33.30941) (width 0.25) (layer "B.Cu") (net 14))
 (segment (start 153.541967 34.88441) (end 153.541967 33.798014) (width 0.25) (layer "B.Cu") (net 14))
 (segment (start 153.053363 33.30941) (end 149.331967 33.30941) (width 0.25) (layer "B.Cu") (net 14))
 (via (at 147.286967 33.80441) (size 0.8) (drill 0.4) (layers "F.Cu" "B.Cu") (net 15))
 (segment (start 153.041967 34.88441) (end 153.041967 33.93441) (width 0.25) (layer "B.Cu") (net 15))
 (segment (start 152.911967 33.80441) (end 147.286967 33.80441) (width 0.25) (layer "B.Cu") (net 15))
 (segment (start 153.041967 33.93441) (end 152.911967 33.80441) (width 0.25) (layer "B.Cu") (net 15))
 (via (at 147.286967 36.34441) (size 0.8) (drill 0.4) (layers "F.Cu" "B.Cu") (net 16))
 (segment (start 151.911967 34.25441) (end 149.376967 34.25441) (width 0.25) (layer "B.Cu") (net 16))
 (segment (start 149.376967 34.25441) (end 147.286967 36.34441) (width 0.25) (layer "B.Cu") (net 16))
 (segment (start 152.541967 34.88441) (end 151.911967 34.25441) (width 0.25) (layer "B.Cu") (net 16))
 (via (at 147.286967 43.96441) (size 0.8) (drill 0.4) (layers "F.Cu" "B.Cu") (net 3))
 (segment (start 147.433967 43.81741) (end 147.286967 43.96441) (width 0.4) (layer "B.Cu") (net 3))
 (segment (start 161.19441 46.28441) (end 158.72741 43.81741) (width 0.4) (layer "B.Cu") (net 3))
 (segment (start 154.33 43.81741) (end 147.433967 43.81741) (width 0.4) (layer "B.Cu") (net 3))
 (segment (start 154.271967 44.91741) (end 154.271967 43.875443) (width 0.25) (layer "B.Cu") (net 3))
 (segment (start 153.988124 44.91741) (end 154.271967 44.91741) (width 0.25) (layer "B.Cu") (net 3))
 (segment (start 158.72741 43.81741) (end 154.33 43.81741) (width 0.4) (layer "B.Cu") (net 3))
 (segment (start 153.741967 45.163567) (end 153.988124 44.91741) (width 0.25) (layer "B.Cu") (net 3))
 (segment (start 153.741967 46.96441) (end 153.741967 45.163567) (width 0.25) (layer "B.Cu") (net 3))
 (segment (start 167.291967 46.28441) (end 161.19441 46.28441) (width 0.4) (layer "B.Cu") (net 3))
 (segment (start 154.271967 43.875443) (end 154.33 43.81741) (width 0.25) (layer "B.Cu") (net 3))
 (segment (start 160.71 41.11) (end 160.71 39.535534) (width 0.4) (layer "B.Cu") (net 1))
 (segment (start 143.041967 45.94941) (end 145.961377 43.03) (width 0.4) (layer "B.Cu") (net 1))
 (segment (start 160.71 39.535534) (end 160.350876 39.17641) (width 0.4) (layer "B.Cu") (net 1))
 (segment (start 160.350876 39.17641) (end 160.011967 39.17641) (width 0.4) (layer "B.Cu") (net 1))
 (segment (start 145.961377 43.03) (end 158.79 43.03) (width 0.4) (layer "B.Cu") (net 1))
 (segment (start 158.79 43.03) (end 160.71 41.11) (width 0.4) (layer "B.Cu") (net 1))
 (segment (start 143.041967 46.34941) (end 143.041967 45.94941) (width 0.4) (layer "B.Cu") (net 1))
 (segment (start 158.291967 48.40441) (end 158.366967 48.32941) (width 0.25) (layer "B.Cu") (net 8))
 (segment (start 157.09581 44.91741) (end 156.811967 44.91741) (width 0.25) (layer "B.Cu") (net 8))
 (segment (start 157.341967 48.40441) (end 158.291967 48.40441) (width 0.25) (layer "B.Cu") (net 8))
 (segment (start 158.366967 46.188567) (end 157.09581 44.91741) (width 0.25) (layer "B.Cu") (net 8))
 (segment (start 153.741967 48.40441) (end 157.341967 48.40441) (width 0.25) (layer "B.Cu") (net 8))
 (segment (start 158.366967 48.32941) (end 158.366967 46.188567) (width 0.25) (layer "B.Cu") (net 8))
 (segment (start 148.99941 45.19941) (end 145.691967 45.19941) (width 0.4) (layer "B.Cu") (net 2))
 (segment (start 150.06 47.66) (end 150.06 46.26) (width 0.4) (layer "B.Cu") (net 2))
 (segment (start 167.291967 48.28441) (end 166.166377 49.41) (width 0.4) (layer "B.Cu") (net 2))
 (segment (start 151.81 49.41) (end 150.06 47.66) (width 0.4) (layer "B.Cu") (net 2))
 (segment (start 150.06 46.26) (end 148.99941 45.19941) (width 0.4) (layer "B.Cu") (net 2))
 (segment (start 145.691967 45.19941) (end 144.541967 46.34941) (width 0.4) (layer "B.Cu") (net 2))
 (segment (start 166.166377 49.41) (end 151.81 49.41) (width 0.4) (layer "B.Cu") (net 2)))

